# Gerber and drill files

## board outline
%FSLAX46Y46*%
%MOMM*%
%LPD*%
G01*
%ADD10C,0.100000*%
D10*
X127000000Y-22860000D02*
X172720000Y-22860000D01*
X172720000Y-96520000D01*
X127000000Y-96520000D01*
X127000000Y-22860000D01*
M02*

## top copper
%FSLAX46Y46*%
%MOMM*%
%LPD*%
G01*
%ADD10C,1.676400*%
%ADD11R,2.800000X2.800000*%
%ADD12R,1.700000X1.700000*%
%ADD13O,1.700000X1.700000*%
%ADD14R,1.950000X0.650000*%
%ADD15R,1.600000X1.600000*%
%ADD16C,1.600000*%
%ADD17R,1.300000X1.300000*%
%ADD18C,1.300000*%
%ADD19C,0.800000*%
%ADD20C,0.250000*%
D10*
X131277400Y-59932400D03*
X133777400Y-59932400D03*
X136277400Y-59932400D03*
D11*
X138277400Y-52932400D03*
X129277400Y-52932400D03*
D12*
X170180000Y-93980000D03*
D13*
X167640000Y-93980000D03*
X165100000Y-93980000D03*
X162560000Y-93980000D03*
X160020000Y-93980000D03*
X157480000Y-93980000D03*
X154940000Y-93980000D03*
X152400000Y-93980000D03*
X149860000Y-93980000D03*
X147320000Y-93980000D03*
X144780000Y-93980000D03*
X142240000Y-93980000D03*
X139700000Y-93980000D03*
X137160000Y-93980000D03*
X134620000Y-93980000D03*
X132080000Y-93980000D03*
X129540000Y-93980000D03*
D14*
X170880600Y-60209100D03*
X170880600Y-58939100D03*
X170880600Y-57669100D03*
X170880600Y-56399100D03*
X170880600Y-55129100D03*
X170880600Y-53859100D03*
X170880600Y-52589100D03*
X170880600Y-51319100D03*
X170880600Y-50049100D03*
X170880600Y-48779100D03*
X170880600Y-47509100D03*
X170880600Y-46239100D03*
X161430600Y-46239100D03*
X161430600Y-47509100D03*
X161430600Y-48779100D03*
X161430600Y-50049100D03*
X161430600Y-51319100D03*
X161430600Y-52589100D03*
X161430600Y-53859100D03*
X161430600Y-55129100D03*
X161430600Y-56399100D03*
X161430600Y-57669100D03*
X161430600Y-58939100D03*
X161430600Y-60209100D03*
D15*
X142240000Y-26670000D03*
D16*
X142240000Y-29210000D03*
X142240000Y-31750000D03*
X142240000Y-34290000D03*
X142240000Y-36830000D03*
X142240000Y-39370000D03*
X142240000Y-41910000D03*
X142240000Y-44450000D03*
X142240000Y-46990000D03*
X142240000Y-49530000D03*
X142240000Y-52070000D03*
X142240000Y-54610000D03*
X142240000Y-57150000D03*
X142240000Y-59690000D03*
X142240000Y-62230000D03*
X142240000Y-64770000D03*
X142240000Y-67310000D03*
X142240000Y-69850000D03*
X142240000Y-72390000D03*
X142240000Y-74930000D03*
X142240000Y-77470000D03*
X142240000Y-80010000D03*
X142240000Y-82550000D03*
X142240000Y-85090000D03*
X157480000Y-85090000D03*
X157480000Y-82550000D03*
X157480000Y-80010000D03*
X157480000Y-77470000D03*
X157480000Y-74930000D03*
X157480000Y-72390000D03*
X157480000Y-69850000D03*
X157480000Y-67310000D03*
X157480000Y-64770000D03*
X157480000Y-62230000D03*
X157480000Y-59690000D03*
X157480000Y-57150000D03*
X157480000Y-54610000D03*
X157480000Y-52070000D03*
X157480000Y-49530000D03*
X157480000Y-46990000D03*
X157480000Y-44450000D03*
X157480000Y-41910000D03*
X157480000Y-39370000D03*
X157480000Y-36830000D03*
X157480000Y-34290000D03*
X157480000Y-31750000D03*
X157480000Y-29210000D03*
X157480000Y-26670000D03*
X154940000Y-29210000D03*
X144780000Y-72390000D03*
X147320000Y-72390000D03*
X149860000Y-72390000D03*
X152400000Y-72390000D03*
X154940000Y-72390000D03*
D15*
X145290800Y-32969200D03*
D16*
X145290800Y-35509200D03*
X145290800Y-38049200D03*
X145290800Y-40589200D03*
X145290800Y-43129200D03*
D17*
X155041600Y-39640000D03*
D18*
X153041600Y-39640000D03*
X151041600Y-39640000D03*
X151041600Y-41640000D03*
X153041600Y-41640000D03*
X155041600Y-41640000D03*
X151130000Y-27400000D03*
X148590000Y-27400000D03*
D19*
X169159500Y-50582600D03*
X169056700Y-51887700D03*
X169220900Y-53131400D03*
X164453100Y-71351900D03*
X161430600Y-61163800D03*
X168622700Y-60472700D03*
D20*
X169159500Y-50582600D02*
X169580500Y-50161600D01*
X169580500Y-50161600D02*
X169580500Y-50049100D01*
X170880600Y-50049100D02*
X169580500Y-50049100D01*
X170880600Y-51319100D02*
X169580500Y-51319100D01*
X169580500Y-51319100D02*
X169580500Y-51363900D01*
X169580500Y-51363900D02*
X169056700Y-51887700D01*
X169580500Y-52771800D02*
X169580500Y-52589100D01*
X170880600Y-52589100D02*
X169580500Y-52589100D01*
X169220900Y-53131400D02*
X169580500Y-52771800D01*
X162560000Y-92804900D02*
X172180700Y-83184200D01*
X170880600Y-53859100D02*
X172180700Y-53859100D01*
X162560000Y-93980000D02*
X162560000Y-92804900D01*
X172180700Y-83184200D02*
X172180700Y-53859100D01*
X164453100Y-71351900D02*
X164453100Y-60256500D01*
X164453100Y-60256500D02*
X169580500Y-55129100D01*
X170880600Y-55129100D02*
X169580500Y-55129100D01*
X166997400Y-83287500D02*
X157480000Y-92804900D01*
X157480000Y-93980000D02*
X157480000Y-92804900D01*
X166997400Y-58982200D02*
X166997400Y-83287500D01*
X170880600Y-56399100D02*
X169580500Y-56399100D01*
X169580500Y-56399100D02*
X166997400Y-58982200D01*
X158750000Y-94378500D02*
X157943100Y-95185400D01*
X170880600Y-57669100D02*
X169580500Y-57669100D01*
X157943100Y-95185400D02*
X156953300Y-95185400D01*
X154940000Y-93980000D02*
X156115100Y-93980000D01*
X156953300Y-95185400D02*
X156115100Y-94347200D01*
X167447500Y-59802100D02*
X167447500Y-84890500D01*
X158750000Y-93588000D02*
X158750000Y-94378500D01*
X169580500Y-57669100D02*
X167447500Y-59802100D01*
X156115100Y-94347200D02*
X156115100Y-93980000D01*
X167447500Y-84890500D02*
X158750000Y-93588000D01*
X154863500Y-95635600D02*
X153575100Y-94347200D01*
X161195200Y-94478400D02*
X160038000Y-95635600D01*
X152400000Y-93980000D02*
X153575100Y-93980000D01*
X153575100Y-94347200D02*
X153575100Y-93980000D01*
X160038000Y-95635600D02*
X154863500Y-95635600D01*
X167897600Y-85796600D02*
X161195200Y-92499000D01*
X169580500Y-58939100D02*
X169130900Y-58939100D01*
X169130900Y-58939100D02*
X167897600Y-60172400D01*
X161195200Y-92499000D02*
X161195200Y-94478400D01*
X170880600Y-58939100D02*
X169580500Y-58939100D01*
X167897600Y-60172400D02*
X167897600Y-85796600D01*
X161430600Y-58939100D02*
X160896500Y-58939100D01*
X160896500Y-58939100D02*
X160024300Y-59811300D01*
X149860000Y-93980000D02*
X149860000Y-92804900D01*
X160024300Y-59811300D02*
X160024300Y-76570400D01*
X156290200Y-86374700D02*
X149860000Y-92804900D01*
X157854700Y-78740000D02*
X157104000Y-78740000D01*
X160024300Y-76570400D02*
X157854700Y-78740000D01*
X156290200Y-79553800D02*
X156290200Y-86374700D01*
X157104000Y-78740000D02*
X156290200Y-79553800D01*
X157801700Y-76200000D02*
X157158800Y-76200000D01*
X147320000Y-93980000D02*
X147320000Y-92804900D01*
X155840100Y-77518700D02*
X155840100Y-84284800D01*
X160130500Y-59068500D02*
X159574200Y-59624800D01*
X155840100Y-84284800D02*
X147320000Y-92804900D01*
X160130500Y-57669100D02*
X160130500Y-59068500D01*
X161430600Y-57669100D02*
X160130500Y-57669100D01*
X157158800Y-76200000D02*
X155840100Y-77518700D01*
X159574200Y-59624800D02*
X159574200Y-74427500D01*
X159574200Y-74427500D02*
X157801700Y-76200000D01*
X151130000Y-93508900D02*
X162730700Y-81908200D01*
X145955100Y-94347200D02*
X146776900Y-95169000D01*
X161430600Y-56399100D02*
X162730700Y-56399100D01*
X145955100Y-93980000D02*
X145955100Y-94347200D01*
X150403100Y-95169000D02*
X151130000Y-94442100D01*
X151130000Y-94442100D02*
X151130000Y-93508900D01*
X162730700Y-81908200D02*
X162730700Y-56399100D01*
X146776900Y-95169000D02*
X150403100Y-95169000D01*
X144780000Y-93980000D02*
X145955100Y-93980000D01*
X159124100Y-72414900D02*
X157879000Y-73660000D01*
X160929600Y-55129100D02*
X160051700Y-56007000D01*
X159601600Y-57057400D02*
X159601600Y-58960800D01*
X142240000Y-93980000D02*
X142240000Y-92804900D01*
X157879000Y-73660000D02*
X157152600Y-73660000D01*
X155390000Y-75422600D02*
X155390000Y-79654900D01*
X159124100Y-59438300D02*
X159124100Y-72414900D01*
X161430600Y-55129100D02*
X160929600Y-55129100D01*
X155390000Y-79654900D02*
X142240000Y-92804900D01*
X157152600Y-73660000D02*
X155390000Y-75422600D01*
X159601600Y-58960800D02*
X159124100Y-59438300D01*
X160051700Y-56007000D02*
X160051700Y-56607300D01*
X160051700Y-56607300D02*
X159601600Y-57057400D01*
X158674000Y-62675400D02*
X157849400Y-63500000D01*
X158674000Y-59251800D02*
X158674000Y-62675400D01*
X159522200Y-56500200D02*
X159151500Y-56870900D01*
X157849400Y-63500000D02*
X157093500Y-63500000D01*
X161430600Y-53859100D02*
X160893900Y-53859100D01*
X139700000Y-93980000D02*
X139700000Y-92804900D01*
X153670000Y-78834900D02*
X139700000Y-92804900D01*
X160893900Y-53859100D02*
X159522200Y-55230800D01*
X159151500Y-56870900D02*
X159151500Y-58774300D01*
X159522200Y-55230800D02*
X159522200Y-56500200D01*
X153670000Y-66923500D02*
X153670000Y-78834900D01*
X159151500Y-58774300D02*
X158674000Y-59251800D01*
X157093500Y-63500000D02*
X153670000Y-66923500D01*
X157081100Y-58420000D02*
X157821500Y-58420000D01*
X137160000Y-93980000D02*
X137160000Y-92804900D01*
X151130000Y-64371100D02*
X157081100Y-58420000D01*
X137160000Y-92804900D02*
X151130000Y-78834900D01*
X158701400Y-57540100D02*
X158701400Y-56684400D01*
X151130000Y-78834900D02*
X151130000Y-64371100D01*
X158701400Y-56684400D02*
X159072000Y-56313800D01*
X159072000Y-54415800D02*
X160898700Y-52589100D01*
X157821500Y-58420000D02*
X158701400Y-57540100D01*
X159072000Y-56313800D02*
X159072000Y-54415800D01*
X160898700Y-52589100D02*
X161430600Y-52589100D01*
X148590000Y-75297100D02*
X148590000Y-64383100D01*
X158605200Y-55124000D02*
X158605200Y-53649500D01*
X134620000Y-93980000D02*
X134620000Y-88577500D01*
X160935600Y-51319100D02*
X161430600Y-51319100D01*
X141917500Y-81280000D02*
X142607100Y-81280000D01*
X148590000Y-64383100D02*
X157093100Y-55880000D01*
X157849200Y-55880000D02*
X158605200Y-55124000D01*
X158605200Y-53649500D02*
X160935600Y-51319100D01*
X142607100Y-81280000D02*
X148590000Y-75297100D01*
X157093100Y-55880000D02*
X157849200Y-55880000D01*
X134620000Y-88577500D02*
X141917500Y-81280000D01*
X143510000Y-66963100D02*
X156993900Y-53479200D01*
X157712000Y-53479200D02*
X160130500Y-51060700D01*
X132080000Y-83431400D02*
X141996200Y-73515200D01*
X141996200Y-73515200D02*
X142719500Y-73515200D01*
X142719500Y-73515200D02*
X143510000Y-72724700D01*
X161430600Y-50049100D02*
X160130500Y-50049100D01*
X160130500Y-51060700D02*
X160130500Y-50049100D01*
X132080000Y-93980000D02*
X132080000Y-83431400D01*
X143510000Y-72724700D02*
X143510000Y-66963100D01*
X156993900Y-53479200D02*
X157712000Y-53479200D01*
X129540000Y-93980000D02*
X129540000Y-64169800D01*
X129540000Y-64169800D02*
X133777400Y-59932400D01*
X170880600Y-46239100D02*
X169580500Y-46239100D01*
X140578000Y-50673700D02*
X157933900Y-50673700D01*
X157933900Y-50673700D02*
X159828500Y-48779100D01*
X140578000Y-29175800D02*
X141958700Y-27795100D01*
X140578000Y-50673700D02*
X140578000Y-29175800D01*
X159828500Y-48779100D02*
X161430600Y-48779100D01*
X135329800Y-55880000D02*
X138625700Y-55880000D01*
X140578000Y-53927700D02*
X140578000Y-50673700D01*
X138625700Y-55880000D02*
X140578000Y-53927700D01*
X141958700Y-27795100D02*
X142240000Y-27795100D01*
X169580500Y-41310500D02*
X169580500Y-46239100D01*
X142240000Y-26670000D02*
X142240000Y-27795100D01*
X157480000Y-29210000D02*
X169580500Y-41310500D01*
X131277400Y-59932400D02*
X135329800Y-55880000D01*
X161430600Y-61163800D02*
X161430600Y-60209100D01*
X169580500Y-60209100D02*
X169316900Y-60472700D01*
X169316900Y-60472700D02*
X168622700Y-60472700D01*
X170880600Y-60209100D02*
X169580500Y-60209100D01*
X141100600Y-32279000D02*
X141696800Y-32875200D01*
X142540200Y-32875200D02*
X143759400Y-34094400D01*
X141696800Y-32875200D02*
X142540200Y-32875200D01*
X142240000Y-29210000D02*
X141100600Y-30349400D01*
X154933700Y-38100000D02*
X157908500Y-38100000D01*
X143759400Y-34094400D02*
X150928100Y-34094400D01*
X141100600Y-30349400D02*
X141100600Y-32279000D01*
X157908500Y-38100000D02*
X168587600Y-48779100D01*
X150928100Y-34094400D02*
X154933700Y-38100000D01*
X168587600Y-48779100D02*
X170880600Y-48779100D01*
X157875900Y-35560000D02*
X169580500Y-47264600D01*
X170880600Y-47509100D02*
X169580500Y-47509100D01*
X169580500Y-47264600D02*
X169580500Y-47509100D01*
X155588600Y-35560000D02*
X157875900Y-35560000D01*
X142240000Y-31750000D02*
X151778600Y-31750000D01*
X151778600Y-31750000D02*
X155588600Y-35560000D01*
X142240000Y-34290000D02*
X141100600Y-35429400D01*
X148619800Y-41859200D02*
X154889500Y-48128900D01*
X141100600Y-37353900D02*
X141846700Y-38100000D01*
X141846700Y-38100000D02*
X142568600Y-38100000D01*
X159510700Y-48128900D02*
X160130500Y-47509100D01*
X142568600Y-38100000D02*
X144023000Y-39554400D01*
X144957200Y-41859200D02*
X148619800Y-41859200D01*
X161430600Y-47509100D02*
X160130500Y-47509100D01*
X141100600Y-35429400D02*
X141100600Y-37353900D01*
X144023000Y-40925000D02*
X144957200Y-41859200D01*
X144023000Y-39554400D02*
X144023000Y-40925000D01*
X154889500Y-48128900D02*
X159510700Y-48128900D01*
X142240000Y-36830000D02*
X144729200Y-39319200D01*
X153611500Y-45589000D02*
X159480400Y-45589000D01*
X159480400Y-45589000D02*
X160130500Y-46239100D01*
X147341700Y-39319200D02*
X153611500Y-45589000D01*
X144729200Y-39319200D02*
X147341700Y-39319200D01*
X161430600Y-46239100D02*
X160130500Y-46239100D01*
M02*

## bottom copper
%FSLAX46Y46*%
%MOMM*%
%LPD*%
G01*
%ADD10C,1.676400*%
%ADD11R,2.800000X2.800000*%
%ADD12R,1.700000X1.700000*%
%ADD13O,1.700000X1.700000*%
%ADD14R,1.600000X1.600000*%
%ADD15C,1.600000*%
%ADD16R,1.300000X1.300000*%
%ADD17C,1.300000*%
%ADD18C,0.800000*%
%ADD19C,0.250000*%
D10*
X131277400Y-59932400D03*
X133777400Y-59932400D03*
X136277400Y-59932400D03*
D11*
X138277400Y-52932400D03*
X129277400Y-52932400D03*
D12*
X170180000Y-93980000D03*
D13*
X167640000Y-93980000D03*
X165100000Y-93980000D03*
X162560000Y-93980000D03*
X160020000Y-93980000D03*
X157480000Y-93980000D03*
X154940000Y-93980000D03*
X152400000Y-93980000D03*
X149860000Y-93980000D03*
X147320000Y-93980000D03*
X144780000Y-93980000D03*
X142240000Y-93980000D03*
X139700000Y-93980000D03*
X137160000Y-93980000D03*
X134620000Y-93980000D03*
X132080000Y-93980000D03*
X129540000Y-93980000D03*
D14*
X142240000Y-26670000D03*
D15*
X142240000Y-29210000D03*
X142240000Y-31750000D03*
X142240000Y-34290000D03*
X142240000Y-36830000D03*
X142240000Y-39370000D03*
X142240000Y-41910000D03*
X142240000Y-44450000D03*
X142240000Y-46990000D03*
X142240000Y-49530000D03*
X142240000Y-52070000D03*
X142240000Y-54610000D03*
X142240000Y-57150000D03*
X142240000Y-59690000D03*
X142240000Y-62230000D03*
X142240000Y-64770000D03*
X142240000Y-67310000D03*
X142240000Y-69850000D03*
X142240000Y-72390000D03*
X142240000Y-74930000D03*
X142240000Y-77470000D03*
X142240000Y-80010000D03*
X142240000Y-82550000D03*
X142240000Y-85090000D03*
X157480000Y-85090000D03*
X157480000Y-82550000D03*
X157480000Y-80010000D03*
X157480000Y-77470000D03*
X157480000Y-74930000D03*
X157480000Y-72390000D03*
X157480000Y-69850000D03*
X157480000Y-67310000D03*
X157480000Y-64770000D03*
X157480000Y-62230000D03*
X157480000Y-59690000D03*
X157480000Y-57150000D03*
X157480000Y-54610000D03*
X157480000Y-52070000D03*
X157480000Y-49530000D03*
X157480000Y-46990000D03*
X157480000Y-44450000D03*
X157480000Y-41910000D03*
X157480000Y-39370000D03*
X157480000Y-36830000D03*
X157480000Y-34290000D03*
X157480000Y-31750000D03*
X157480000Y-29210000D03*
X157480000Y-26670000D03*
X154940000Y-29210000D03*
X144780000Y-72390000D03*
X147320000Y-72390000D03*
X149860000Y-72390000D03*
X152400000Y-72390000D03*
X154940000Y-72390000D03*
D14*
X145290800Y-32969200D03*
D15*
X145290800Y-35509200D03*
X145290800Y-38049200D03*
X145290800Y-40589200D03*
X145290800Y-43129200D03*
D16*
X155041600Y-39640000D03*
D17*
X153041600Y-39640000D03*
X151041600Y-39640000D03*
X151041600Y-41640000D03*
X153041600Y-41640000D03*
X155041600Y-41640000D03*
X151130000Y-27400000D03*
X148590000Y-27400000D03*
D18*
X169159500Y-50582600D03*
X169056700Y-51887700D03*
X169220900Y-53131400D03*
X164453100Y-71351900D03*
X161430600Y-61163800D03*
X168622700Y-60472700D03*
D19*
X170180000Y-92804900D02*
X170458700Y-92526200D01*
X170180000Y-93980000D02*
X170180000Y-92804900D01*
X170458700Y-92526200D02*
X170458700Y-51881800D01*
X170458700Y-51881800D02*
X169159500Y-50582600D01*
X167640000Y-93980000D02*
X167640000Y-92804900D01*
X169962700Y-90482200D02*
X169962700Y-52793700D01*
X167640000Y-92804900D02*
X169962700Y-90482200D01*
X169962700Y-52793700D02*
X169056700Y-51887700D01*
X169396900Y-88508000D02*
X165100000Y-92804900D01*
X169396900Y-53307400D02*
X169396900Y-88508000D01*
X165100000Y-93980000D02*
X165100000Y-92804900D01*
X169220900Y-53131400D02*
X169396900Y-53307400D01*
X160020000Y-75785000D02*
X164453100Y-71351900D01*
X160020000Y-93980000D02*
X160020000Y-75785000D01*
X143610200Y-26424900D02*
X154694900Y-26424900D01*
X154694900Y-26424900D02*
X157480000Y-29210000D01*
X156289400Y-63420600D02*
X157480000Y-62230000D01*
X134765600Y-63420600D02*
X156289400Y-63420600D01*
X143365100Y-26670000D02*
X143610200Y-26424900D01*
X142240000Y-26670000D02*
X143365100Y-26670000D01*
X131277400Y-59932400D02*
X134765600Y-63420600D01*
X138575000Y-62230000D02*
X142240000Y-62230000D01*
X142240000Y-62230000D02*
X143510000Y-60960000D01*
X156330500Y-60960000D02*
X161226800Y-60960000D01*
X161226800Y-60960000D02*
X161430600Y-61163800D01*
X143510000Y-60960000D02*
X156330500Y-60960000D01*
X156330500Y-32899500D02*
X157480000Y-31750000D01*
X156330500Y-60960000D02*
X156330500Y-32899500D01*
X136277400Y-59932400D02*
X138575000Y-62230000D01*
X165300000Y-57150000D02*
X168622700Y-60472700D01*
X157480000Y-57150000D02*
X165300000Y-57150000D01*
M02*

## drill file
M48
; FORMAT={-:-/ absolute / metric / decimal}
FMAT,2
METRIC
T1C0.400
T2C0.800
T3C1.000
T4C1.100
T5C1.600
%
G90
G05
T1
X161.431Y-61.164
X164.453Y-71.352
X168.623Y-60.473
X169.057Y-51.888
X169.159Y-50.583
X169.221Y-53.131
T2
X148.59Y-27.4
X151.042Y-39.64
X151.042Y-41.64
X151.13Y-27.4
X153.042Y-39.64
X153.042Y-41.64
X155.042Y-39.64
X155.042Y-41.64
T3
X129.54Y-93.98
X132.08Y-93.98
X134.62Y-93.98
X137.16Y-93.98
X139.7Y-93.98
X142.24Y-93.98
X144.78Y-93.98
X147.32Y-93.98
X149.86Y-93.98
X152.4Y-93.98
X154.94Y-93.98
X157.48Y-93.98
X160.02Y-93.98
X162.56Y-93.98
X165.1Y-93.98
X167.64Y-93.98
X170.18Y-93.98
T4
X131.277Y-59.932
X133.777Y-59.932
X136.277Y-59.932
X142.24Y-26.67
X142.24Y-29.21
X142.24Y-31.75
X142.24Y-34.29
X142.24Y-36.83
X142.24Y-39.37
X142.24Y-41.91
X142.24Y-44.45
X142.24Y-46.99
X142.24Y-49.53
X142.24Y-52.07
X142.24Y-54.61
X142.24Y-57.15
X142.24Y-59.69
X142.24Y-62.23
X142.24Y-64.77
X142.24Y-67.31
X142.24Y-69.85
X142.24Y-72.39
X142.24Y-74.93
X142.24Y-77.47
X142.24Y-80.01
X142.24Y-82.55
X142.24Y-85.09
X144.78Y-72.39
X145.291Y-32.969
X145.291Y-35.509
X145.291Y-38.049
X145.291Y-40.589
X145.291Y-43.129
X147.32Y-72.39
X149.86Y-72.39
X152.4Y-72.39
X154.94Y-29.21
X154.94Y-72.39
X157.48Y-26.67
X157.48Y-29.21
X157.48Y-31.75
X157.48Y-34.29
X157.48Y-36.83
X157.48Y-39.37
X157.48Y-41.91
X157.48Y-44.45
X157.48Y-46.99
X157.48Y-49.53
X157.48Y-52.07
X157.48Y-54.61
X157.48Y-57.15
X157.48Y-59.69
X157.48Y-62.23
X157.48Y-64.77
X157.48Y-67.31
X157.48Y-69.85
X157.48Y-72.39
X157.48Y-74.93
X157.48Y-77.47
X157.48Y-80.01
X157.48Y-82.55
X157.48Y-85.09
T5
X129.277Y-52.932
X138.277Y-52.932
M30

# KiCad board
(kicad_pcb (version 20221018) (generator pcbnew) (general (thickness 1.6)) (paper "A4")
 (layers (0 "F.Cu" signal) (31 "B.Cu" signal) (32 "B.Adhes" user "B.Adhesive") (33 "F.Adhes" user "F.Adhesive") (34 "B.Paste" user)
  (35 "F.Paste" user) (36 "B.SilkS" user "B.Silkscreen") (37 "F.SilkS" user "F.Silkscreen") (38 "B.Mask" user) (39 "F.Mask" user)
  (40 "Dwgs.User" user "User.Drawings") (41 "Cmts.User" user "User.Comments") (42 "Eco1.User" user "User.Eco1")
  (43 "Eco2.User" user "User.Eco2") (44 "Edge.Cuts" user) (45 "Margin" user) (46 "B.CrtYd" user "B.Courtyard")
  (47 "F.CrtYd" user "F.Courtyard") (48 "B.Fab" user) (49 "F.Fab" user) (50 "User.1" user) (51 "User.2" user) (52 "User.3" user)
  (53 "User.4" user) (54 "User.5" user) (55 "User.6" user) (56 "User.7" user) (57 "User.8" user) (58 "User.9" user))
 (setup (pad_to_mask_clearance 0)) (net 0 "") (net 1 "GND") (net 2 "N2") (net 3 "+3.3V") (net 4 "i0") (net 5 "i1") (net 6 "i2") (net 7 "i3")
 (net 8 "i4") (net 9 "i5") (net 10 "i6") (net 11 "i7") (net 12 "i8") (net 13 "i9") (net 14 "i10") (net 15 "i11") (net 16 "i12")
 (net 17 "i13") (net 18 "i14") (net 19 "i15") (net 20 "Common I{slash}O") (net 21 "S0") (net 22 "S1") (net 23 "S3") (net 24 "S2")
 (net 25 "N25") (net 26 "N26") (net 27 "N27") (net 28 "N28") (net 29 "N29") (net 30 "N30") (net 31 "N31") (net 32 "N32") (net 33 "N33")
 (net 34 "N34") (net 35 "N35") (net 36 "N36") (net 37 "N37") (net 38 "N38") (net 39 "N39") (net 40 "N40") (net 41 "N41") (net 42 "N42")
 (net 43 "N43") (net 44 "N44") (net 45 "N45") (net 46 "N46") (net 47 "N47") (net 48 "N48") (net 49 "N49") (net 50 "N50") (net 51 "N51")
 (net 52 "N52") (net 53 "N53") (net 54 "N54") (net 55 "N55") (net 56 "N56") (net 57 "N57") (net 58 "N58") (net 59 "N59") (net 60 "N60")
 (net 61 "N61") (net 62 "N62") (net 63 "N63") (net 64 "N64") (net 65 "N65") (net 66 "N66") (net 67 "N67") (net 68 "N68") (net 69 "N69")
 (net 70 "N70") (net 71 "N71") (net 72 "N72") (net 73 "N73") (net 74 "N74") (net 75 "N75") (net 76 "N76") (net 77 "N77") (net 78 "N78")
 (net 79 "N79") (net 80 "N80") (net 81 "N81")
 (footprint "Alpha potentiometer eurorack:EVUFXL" (layer "F.Cu") (at 133.7774 52.9324)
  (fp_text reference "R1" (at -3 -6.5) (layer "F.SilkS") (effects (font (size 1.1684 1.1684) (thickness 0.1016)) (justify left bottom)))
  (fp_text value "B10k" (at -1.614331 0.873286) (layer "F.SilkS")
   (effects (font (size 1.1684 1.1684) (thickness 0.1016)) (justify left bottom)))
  (pad "1" thru_hole circle (at -2.5 7 270) (size 1.6764 1.6764) (drill 1.1) (layers "*.Cu" "*.Mask") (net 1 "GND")
   (solder_mask_margin 0.1016))
  (pad "2" thru_hole circle (at 0 7 270) (size 1.6764 1.6764) (drill 1.1) (layers "*.Cu" "*.Mask") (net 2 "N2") (solder_mask_margin 0.1016))
  (pad "3" thru_hole circle (at 2.5 7 270) (size 1.6764 1.6764) (drill 1.1) (layers "*.Cu" "*.Mask") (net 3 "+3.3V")
   (solder_mask_margin 0.1016))
  (pad "M1" thru_hole rect (at 4.5 0 270) (size 2.8 2.8) (drill 1.6) (layers "*.Cu" "*.Mask") (solder_mask_margin 0.1016)
   (thermal_bridge_angle 45))
  (pad "M2" thru_hole rect (at -4.5 0 270) (size 2.8 2.8) (drill 1.6) (layers "*.Cu" "*.Mask") (solder_mask_margin 0.1016)
   (thermal_bridge_angle 45)))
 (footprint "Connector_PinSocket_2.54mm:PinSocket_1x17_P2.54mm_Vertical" (layer "F.Cu") (at 170.18 93.98 -90)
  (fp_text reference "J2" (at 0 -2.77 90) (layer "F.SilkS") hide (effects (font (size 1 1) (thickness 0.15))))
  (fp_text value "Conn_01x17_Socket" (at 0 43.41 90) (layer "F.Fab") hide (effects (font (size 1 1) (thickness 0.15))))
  (pad "1" thru_hole rect (at 0 0 270) (size 1.7 1.7) (drill 1) (layers "*.Cu" "*.Mask") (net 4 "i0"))
  (pad "2" thru_hole oval (at 0 2.54 270) (size 1.7 1.7) (drill 1) (layers "*.Cu" "*.Mask") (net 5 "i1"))
  (pad "3" thru_hole oval (at 0 5.08 270) (size 1.7 1.7) (drill 1) (layers "*.Cu" "*.Mask") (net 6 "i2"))
  (pad "4" thru_hole oval (at 0 7.62 270) (size 1.7 1.7) (drill 1) (layers "*.Cu" "*.Mask") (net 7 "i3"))
  (pad "5" thru_hole oval (at 0 10.16 270) (size 1.7 1.7) (drill 1) (layers "*.Cu" "*.Mask") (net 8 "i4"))
  (pad "6" thru_hole oval (at 0 12.7 270) (size 1.7 1.7) (drill 1) (layers "*.Cu" "*.Mask") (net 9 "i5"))
  (pad "7" thru_hole oval (at 0 15.24 270) (size 1.7 1.7) (drill 1) (layers "*.Cu" "*.Mask") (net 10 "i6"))
  (pad "8" thru_hole oval (at 0 17.78 270) (size 1.7 1.7) (drill 1) (layers "*.Cu" "*.Mask") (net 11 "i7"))
  (pad "9" thru_hole oval (at 0 20.32 270) (size 1.7 1.7) (drill 1) (layers "*.Cu" "*.Mask") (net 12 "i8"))
  (pad "10" thru_hole oval (at 0 22.86 270) (size 1.7 1.7) (drill 1) (layers "*.Cu" "*.Mask") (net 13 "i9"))
  (pad "11" thru_hole oval (at 0 25.4 270) (size 1.7 1.7) (drill 1) (layers "*.Cu" "*.Mask") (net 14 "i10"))
  (pad "12" thru_hole oval (at 0 27.94 270) (size 1.7 1.7) (drill 1) (layers "*.Cu" "*.Mask") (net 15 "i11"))
  (pad "13" thru_hole oval (at 0 30.48 270) (size 1.7 1.7) (drill 1) (layers "*.Cu" "*.Mask") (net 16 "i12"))
  (pad "14" thru_hole oval (at 0 33.02 270) (size 1.7 1.7) (drill 1) (layers "*.Cu" "*.Mask") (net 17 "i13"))
  (pad "15" thru_hole oval (at 0 35.56 270) (size 1.7 1.7) (drill 1) (layers "*.Cu" "*.Mask") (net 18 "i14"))
  (pad "16" thru_hole oval (at 0 38.1 270) (size 1.7 1.7) (drill 1) (layers "*.Cu" "*.Mask") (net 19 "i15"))
  (pad "17" thru_hole oval (at 0 40.64 270) (size 1.7 1.7) (drill 1) (layers "*.Cu" "*.Mask") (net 2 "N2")))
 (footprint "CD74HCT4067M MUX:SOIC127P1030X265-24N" (layer "F.Cu") (at 166.1556 53.2241 180)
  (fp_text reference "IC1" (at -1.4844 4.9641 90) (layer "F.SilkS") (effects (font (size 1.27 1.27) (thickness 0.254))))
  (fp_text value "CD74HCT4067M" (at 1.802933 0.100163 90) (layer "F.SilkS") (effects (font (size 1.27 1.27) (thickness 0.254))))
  (pad "1" smd rect (at -4.725 -6.985 270) (size 0.65 1.95) (layers "F.Cu" "F.Paste" "F.Mask") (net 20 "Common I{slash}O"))
  (pad "2" smd rect (at -4.725 -5.715 270) (size 0.65 1.95) (layers "F.Cu" "F.Paste" "F.Mask") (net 11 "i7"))
  (pad "3" smd rect (at -4.725 -4.445 270) (size 0.65 1.95) (layers "F.Cu" "F.Paste" "F.Mask") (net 10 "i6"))
  (pad "4" smd rect (at -4.725 -3.175 270) (size 0.65 1.95) (layers "F.Cu" "F.Paste" "F.Mask") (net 9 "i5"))
  (pad "5" smd rect (at -4.725 -1.905 270) (size 0.65 1.95) (layers "F.Cu" "F.Paste" "F.Mask") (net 8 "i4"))
  (pad "6" smd rect (at -4.725 -0.635 270) (size 0.65 1.95) (layers "F.Cu" "F.Paste" "F.Mask") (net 7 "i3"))
  (pad "7" smd rect (at -4.725 0.635 270) (size 0.65 1.95) (layers "F.Cu" "F.Paste" "F.Mask") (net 6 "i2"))
  (pad "8" smd rect (at -4.725 1.905 270) (size 0.65 1.95) (layers "F.Cu" "F.Paste" "F.Mask") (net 5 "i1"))
  (pad "9" smd rect (at -4.725 3.175 270) (size 0.65 1.95) (layers "F.Cu" "F.Paste" "F.Mask") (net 4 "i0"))
  (pad "10" smd rect (at -4.725 4.445 270) (size 0.65 1.95) (layers "F.Cu" "F.Paste" "F.Mask") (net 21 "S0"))
  (pad "11" smd rect (at -4.725 5.715 270) (size 0.65 1.95) (layers "F.Cu" "F.Paste" "F.Mask") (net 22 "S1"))
  (pad "12" smd rect (at -4.725 6.985 270) (size 0.65 1.95) (layers "F.Cu" "F.Paste" "F.Mask") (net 1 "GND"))
  (pad "13" smd rect (at 4.725 6.985 270) (size 0.65 1.95) (layers "F.Cu" "F.Paste" "F.Mask") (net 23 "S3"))
  (pad "14" smd rect (at 4.725 5.715 270) (size 0.65 1.95) (layers "F.Cu" "F.Paste" "F.Mask") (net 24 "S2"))
  (pad "15" smd rect (at 4.725 4.445 270) (size 0.65 1.95) (layers "F.Cu" "F.Paste" "F.Mask") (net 1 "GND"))
  (pad "16" smd rect (at 4.725 3.175 270) (size 0.65 1.95) (layers "F.Cu" "F.Paste" "F.Mask") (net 19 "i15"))
  (pad "17" smd rect (at 4.725 1.905 270) (size 0.65 1.95) (layers "F.Cu" "F.Paste" "F.Mask") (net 18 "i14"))
  (pad "18" smd rect (at 4.725 0.635 270) (size 0.65 1.95) (layers "F.Cu" "F.Paste" "F.Mask") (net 17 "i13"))
  (pad "19" smd rect (at 4.725 -0.635 270) (size 0.65 1.95) (layers "F.Cu" "F.Paste" "F.Mask") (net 16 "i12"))
  (pad "20" smd rect (at 4.725 -1.905 270) (size 0.65 1.95) (layers "F.Cu" "F.Paste" "F.Mask") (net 15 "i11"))
  (pad "21" smd rect (at 4.725 -3.175 270) (size 0.65 1.95) (layers "F.Cu" "F.Paste" "F.Mask") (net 14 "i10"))
  (pad "22" smd rect (at 4.725 -4.445 270) (size 0.65 1.95) (layers "F.Cu" "F.Paste" "F.Mask") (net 13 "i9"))
  (pad "23" smd rect (at 4.725 -5.715 270) (size 0.65 1.95) (layers "F.Cu" "F.Paste" "F.Mask") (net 12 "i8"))
  (pad "24" smd rect (at 4.725 -6.985 270) (size 0.65 1.95) (layers "F.Cu" "F.Paste" "F.Mask") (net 3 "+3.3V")))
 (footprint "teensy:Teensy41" (layer "F.Cu") (at 149.86 55.88 -90)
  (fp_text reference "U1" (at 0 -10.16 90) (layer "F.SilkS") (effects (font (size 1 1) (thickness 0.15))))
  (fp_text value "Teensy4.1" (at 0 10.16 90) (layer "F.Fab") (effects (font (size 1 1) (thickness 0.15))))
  (pad "1" thru_hole rect (at -29.21 7.62 270) (size 1.6 1.6) (drill 1.1) (layers "*.Cu" "*.Mask") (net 1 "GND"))
  (pad "2" thru_hole circle (at -26.67 7.62 270) (size 1.6 1.6) (drill 1.1) (layers "*.Cu" "*.Mask") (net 21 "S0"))
  (pad "3" thru_hole circle (at -24.13 7.62 270) (size 1.6 1.6) (drill 1.1) (layers "*.Cu" "*.Mask") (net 22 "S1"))
  (pad "4" thru_hole circle (at -21.59 7.62 270) (size 1.6 1.6) (drill 1.1) (layers "*.Cu" "*.Mask") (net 24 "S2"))
  (pad "5" thru_hole circle (at -19.05 7.62 270) (size 1.6 1.6) (drill 1.1) (layers "*.Cu" "*.Mask") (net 23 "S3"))
  (pad "6" thru_hole circle (at -16.51 7.62 270) (size 1.6 1.6) (drill 1.1) (layers "*.Cu" "*.Mask") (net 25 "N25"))
  (pad "7" thru_hole circle (at -13.97 7.62 270) (size 1.6 1.6) (drill 1.1) (layers "*.Cu" "*.Mask") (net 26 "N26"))
  (pad "8" thru_hole circle (at -11.43 7.62 270) (size 1.6 1.6) (drill 1.1) (layers "*.Cu" "*.Mask") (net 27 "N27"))
  (pad "9" thru_hole circle (at -8.89 7.62 270) (size 1.6 1.6) (drill 1.1) (layers "*.Cu" "*.Mask") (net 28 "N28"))
  (pad "10" thru_hole circle (at -6.35 7.62 270) (size 1.6 1.6) (drill 1.1) (layers "*.Cu" "*.Mask") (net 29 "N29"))
  (pad "11" thru_hole circle (at -3.81 7.62 270) (size 1.6 1.6) (drill 1.1) (layers "*.Cu" "*.Mask") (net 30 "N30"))
  (pad "12" thru_hole circle (at -1.27 7.62 270) (size 1.6 1.6) (drill 1.1) (layers "*.Cu" "*.Mask") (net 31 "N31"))
  (pad "13" thru_hole circle (at 1.27 7.62 270) (size 1.6 1.6) (drill 1.1) (layers "*.Cu" "*.Mask") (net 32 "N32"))
  (pad "14" thru_hole circle (at 3.81 7.62 270) (size 1.6 1.6) (drill 1.1) (layers "*.Cu" "*.Mask") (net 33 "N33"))
  (pad "15" thru_hole circle (at 6.35 7.62 270) (size 1.6 1.6) (drill 1.1) (layers "*.Cu" "*.Mask") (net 3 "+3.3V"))
  (pad "16" thru_hole circle (at 8.89 7.62 270) (size 1.6 1.6) (drill 1.1) (layers "*.Cu" "*.Mask") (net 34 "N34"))
  (pad "17" thru_hole circle (at 11.43 7.62 270) (size 1.6 1.6) (drill 1.1) (layers "*.Cu" "*.Mask") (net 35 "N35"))
  (pad "18" thru_hole circle (at 13.97 7.62 270) (size 1.6 1.6) (drill 1.1) (layers "*.Cu" "*.Mask") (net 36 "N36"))
  (pad "19" thru_hole circle (at 16.51 7.62 270) (size 1.6 1.6) (drill 1.1) (layers "*.Cu" "*.Mask") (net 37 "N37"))
  (pad "20" thru_hole circle (at 19.05 7.62 270) (size 1.6 1.6) (drill 1.1) (layers "*.Cu" "*.Mask") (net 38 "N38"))
  (pad "21" thru_hole circle (at 21.59 7.62 270) (size 1.6 1.6) (drill 1.1) (layers "*.Cu" "*.Mask") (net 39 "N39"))
  (pad "22" thru_hole circle (at 24.13 7.62 270) (size 1.6 1.6) (drill 1.1) (layers "*.Cu" "*.Mask") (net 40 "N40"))
  (pad "23" thru_hole circle (at 26.67 7.62 270) (size 1.6 1.6) (drill 1.1) (layers "*.Cu" "*.Mask") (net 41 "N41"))
  (pad "24" thru_hole circle (at 29.21 7.62 270) (size 1.6 1.6) (drill 1.1) (layers "*.Cu" "*.Mask") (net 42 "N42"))
  (pad "25" thru_hole circle (at 29.21 -7.62 270) (size 1.6 1.6) (drill 1.1) (layers "*.Cu" "*.Mask") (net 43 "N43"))
  (pad "26" thru_hole circle (at 26.67 -7.62 270) (size 1.6 1.6) (drill 1.1) (layers "*.Cu" "*.Mask") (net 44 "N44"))
  (pad "27" thru_hole circle (at 24.13 -7.62 270) (size 1.6 1.6) (drill 1.1) (layers "*.Cu" "*.Mask") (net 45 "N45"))
  (pad "28" thru_hole circle (at 21.59 -7.62 270) (size 1.6 1.6) (drill 1.1) (layers "*.Cu" "*.Mask") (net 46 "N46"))
  (pad "29" thru_hole circle (at 19.05 -7.62 270) (size 1.6 1.6) (drill 1.1) (layers "*.Cu" "*.Mask") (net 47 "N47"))
  (pad "30" thru_hole circle (at 16.51 -7.62 270) (size 1.6 1.6) (drill 1.1) (layers "*.Cu" "*.Mask") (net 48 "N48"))
  (pad "31" thru_hole circle (at 13.97 -7.62 270) (size 1.6 1.6) (drill 1.1) (layers "*.Cu" "*.Mask") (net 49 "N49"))
  (pad "32" thru_hole circle (at 11.43 -7.62 270) (size 1.6 1.6) (drill 1.1) (layers "*.Cu" "*.Mask") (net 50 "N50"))
  (pad "33" thru_hole circle (at 8.89 -7.62 270) (size 1.6 1.6) (drill 1.1) (layers "*.Cu" "*.Mask") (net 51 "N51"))
  (pad "34" thru_hole circle (at 6.35 -7.62 270) (size 1.6 1.6) (drill 1.1) (layers "*.Cu" "*.Mask") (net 1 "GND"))
  (pad "35" thru_hole circle (at 3.81 -7.62 270) (size 1.6 1.6) (drill 1.1) (layers "*.Cu" "*.Mask") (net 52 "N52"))
  (pad "36" thru_hole circle (at 1.27 -7.62 270) (size 1.6 1.6) (drill 1.1) (layers "*.Cu" "*.Mask") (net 20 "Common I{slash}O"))
  (pad "37" thru_hole circle (at -1.27 -7.62 270) (size 1.6 1.6) (drill 1.1) (layers "*.Cu" "*.Mask") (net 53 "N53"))
  (pad "38" thru_hole circle (at -3.81 -7.62 270) (size 1.6 1.6) (drill 1.1) (layers "*.Cu" "*.Mask") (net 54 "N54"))
  (pad "39" thru_hole circle (at -6.35 -7.62 270) (size 1.6 1.6) (drill 1.1) (layers "*.Cu" "*.Mask") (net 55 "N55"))
  (pad "40" thru_hole circle (at -8.89 -7.62 270) (size 1.6 1.6) (drill 1.1) (layers "*.Cu" "*.Mask") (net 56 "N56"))
  (pad "41" thru_hole circle (at -11.43 -7.62 270) (size 1.6 1.6) (drill 1.1) (layers "*.Cu" "*.Mask") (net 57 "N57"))
  (pad "42" thru_hole circle (at -13.97 -7.62 270) (size 1.6 1.6) (drill 1.1) (layers "*.Cu" "*.Mask") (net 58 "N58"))
  (pad "43" thru_hole circle (at -16.51 -7.62 270) (size 1.6 1.6) (drill 1.1) (layers "*.Cu" "*.Mask") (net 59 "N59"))
  (pad "44" thru_hole circle (at -19.05 -7.62 270) (size 1.6 1.6) (drill 1.1) (layers "*.Cu" "*.Mask") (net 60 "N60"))
  (pad "45" thru_hole circle (at -21.59 -7.62 270) (size 1.6 1.6) (drill 1.1) (layers "*.Cu" "*.Mask") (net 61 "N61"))
  (pad "46" thru_hole circle (at -24.13 -7.62 270) (size 1.6 1.6) (drill 1.1) (layers "*.Cu" "*.Mask") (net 3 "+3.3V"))
  (pad "47" thru_hole circle (at -26.67 -7.62 270) (size 1.6 1.6) (drill 1.1) (layers "*.Cu" "*.Mask") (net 1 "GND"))
  (pad "48" thru_hole circle (at -29.21 -7.62 270) (size 1.6 1.6) (drill 1.1) (layers "*.Cu" "*.Mask") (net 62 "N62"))
  (pad "49" thru_hole circle (at -26.67 -5.08 270) (size 1.6 1.6) (drill 1.1) (layers "*.Cu" "*.Mask") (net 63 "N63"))
  (pad "50" thru_hole circle (at 16.51 5.08 270) (size 1.6 1.6) (drill 1.1) (layers "*.Cu" "*.Mask") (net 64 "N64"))
  (pad "51" thru_hole circle (at 16.51 2.54 270) (size 1.6 1.6) (drill 1.1) (layers "*.Cu" "*.Mask") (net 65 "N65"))
  (pad "52" thru_hole circle (at 16.51 0 270) (size 1.6 1.6) (drill 1.1) (layers "*.Cu" "*.Mask") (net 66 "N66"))
  (pad "53" thru_hole circle (at 16.51 -2.54 270) (size 1.6 1.6) (drill 1.1) (layers "*.Cu" "*.Mask") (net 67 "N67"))
  (pad "54" thru_hole circle (at 16.51 -5.08 270) (size 1.6 1.6) (drill 1.1) (layers "*.Cu" "*.Mask") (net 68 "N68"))
  (pad "55" thru_hole rect (at -22.9108 4.5692 270) (size 1.6 1.6) (drill 1.1) (layers "*.Cu" "*.Mask") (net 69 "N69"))
  (pad "56" thru_hole circle (at -20.3708 4.5692 270) (size 1.6 1.6) (drill 1.1) (layers "*.Cu" "*.Mask") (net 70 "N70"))
  (pad "57" thru_hole circle (at -17.8308 4.5692 270) (size 1.6 1.6) (drill 1.1) (layers "*.Cu" "*.Mask") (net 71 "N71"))
  (pad "58" thru_hole circle (at -15.2908 4.5692 270) (size 1.6 1.6) (drill 1.1) (layers "*.Cu" "*.Mask") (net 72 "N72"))
  (pad "59" thru_hole circle (at -12.7508 4.5692 270) (size 1.6 1.6) (drill 1.1) (layers "*.Cu" "*.Mask") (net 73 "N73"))
  (pad "60" thru_hole rect (at -16.24 -5.1816 270) (size 1.3 1.3) (drill 0.8) (layers "*.Cu" "*.Mask") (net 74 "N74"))
  (pad "61" thru_hole circle (at -16.24 -3.1816 270) (size 1.3 1.3) (drill 0.8) (layers "*.Cu" "*.Mask") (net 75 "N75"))
  (pad "62" thru_hole circle (at -16.24 -1.1816 270) (size 1.3 1.3) (drill 0.8) (layers "*.Cu" "*.Mask") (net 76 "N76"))
  (pad "63" thru_hole circle (at -14.24 -1.1816 270) (size 1.3 1.3) (drill 0.8) (layers "*.Cu" "*.Mask") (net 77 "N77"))
  (pad "64" thru_hole circle (at -14.24 -3.1816 270) (size 1.3 1.3) (drill 0.8) (layers "*.Cu" "*.Mask") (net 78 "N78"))
  (pad "65" thru_hole circle (at -14.24 -5.1816 270) (size 1.3 1.3) (drill 0.8) (layers "*.Cu" "*.Mask") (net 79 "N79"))
  (pad "66" thru_hole circle (at -28.48 -1.27 270) (size 1.3 1.3) (drill 0.8) (layers "*.Cu" "*.Mask") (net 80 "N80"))
  (pad "67" thru_hole circle (at -28.48 1.27 270) (size 1.3 1.3) (drill 0.8) (layers "*.Cu" "*.Mask") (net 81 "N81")))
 (gr_rect (start 127 22.86) (end 172.72 96.52) (stroke (width 0.1) (type default)) (fill none) (layer "Edge.Cuts"))
 (segment (start 169.1595 50.5826) (end 169.5805 50.1616) (width 0.25) (layer "F.Cu") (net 4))
 (segment (start 169.5805 50.1616) (end 169.5805 50.0491) (width 0.25) (layer "F.Cu") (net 4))
 (segment (start 170.8806 50.0491) (end 169.5805 50.0491) (width 0.25) (layer "F.Cu") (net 4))
 (via (at 169.1595 50.5826) (size 0.8) (drill 0.4) (layers "F.Cu" "B.Cu") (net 4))
 (segment (start 170.18 92.8049) (end 170.4587 92.5262) (width 0.25) (layer "B.Cu") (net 4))
 (segment (start 170.18 93.98) (end 170.18 92.8049) (width 0.25) (layer "B.Cu") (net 4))
 (segment (start 170.4587 92.5262) (end 170.4587 51.8818) (width 0.25) (layer "B.Cu") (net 4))
 (segment (start 170.4587 51.8818) (end 169.1595 50.5826) (width 0.25) (layer "B.Cu") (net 4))
 (segment (start 170.8806 51.3191) (end 169.5805 51.3191) (width 0.25) (layer "F.Cu") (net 5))
 (segment (start 169.5805 51.3191) (end 169.5805 51.3639) (width 0.25) (layer "F.Cu") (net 5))
 (segment (start 169.5805 51.3639) (end 169.0567 51.8877) (width 0.25) (layer "F.Cu") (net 5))
 (via (at 169.0567 51.8877) (size 0.8) (drill 0.4) (layers "F.Cu" "B.Cu") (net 5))
 (segment (start 167.64 93.98) (end 167.64 92.8049) (width 0.25) (layer "B.Cu") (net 5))
 (segment (start 169.9627 90.4822) (end 169.9627 52.7937) (width 0.25) (layer "B.Cu") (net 5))
 (segment (start 167.64 92.8049) (end 169.9627 90.4822) (width 0.25) (layer "B.Cu") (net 5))
 (segment (start 169.9627 52.7937) (end 169.0567 51.8877) (width 0.25) (layer "B.Cu") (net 5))
 (segment (start 169.5805 52.7718) (end 169.5805 52.5891) (width 0.25) (layer "F.Cu") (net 6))
 (segment (start 170.8806 52.5891) (end 169.5805 52.5891) (width 0.25) (layer "F.Cu") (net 6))
 (segment (start 169.2209 53.1314) (end 169.5805 52.7718) (width 0.25) (layer "F.Cu") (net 6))
 (via (at 169.2209 53.1314) (size 0.8) (drill 0.4) (layers "F.Cu" "B.Cu") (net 6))
 (segment (start 169.3969 88.508) (end 165.1 92.8049) (width 0.25) (layer "B.Cu") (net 6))
 (segment (start 169.3969 53.3074) (end 169.3969 88.508) (width 0.25) (layer "B.Cu") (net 6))
 (segment (start 165.1 93.98) (end 165.1 92.8049) (width 0.25) (layer "B.Cu") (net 6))
 (segment (start 169.2209 53.1314) (end 169.3969 53.3074) (width 0.25) (layer "B.Cu") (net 6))
 (segment (start 162.56 92.8049) (end 172.1807 83.1842) (width 0.25) (layer "F.Cu") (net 7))
 (segment (start 170.8806 53.8591) (end 172.1807 53.8591) (width 0.25) (layer "F.Cu") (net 7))
 (segment (start 162.56 93.98) (end 162.56 92.8049) (width 0.25) (layer "F.Cu") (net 7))
 (segment (start 172.1807 83.1842) (end 172.1807 53.8591) (width 0.25) (layer "F.Cu") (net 7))
 (segment (start 164.4531 71.3519) (end 164.4531 60.2565) (width 0.25) (layer "F.Cu") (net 8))
 (segment (start 164.4531 60.2565) (end 169.5805 55.1291) (width 0.25) (layer "F.Cu") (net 8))
 (segment (start 170.8806 55.1291) (end 169.5805 55.1291) (width 0.25) (layer "F.Cu") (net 8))
 (via (at 164.4531 71.3519) (size 0.8) (drill 0.4) (layers "F.Cu" "B.Cu") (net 8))
 (segment (start 160.02 75.785) (end 164.4531 71.3519) (width 0.25) (layer "B.Cu") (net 8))
 (segment (start 160.02 93.98) (end 160.02 75.785) (width 0.25) (layer "B.Cu") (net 8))
 (segment (start 166.9974 83.2875) (end 157.48 92.8049) (width 0.25) (layer "F.Cu") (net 9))
 (segment (start 157.48 93.98) (end 157.48 92.8049) (width 0.25) (layer "F.Cu") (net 9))
 (segment (start 166.9974 58.9822) (end 166.9974 83.2875) (width 0.25) (layer "F.Cu") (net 9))
 (segment (start 170.8806 56.3991) (end 169.5805 56.3991) (width 0.25) (layer "F.Cu") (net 9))
 (segment (start 169.5805 56.3991) (end 166.9974 58.9822) (width 0.25) (layer "F.Cu") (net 9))
 (segment (start 158.75 94.3785) (end 157.9431 95.1854) (width 0.25) (layer "F.Cu") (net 10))
 (segment (start 170.8806 57.6691) (end 169.5805 57.6691) (width 0.25) (layer "F.Cu") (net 10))
 (segment (start 157.9431 95.1854) (end 156.9533 95.1854) (width 0.25) (layer "F.Cu") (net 10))
 (segment (start 154.94 93.98) (end 156.1151 93.98) (width 0.25) (layer "F.Cu") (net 10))
 (segment (start 156.9533 95.1854) (end 156.1151 94.3472) (width 0.25) (layer "F.Cu") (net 10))
 (segment (start 167.4475 59.8021) (end 167.4475 84.8905) (width 0.25) (layer "F.Cu") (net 10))
 (segment (start 158.75 93.588) (end 158.75 94.3785) (width 0.25) (layer "F.Cu") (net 10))
 (segment (start 169.5805 57.6691) (end 167.4475 59.8021) (width 0.25) (layer "F.Cu") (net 10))
 (segment (start 156.1151 94.3472) (end 156.1151 93.98) (width 0.25) (layer "F.Cu") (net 10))
 (segment (start 167.4475 84.8905) (end 158.75 93.588) (width 0.25) (layer "F.Cu") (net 10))
 (segment (start 154.8635 95.6356) (end 153.5751 94.3472) (width 0.25) (layer "F.Cu") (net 11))
 (segment (start 161.1952 94.4784) (end 160.038 95.6356) (width 0.25) (layer "F.Cu") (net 11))
 (segment (start 152.4 93.98) (end 153.5751 93.98) (width 0.25) (layer "F.Cu") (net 11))
 (segment (start 153.5751 94.3472) (end 153.5751 93.98) (width 0.25) (layer "F.Cu") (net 11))
 (segment (start 160.038 95.6356) (end 154.8635 95.6356) (width 0.25) (layer "F.Cu") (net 11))
 (segment (start 167.8976 85.7966) (end 161.1952 92.499) (width 0.25) (layer "F.Cu") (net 11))
 (segment (start 169.5805 58.9391) (end 169.1309 58.9391) (width 0.25) (layer "F.Cu") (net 11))
 (segment (start 169.1309 58.9391) (end 167.8976 60.1724) (width 0.25) (layer "F.Cu") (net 11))
 (segment (start 161.1952 92.499) (end 161.1952 94.4784) (width 0.25) (layer "F.Cu") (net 11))
 (segment (start 170.8806 58.9391) (end 169.5805 58.9391) (width 0.25) (layer "F.Cu") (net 11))
 (segment (start 167.8976 60.1724) (end 167.8976 85.7966) (width 0.25) (layer "F.Cu") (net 11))
 (segment (start 161.4306 58.9391) (end 160.8965 58.9391) (width 0.25) (layer "F.Cu") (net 12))
 (segment (start 160.8965 58.9391) (end 160.0243 59.8113) (width 0.25) (layer "F.Cu") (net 12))
 (segment (start 149.86 93.98) (end 149.86 92.8049) (width 0.25) (layer "F.Cu") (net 12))
 (segment (start 160.0243 59.8113) (end 160.0243 76.5704) (width 0.25) (layer "F.Cu") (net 12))
 (segment (start 156.2902 86.3747) (end 149.86 92.8049) (width 0.25) (layer "F.Cu") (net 12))
 (segment (start 157.8547 78.74) (end 157.104 78.74) (width 0.25) (layer "F.Cu") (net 12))
 (segment (start 160.0243 76.5704) (end 157.8547 78.74) (width 0.25) (layer "F.Cu") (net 12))
 (segment (start 156.2902 79.5538) (end 156.2902 86.3747) (width 0.25) (layer "F.Cu") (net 12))
 (segment (start 157.104 78.74) (end 156.2902 79.5538) (width 0.25) (layer "F.Cu") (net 12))
 (segment (start 157.8017 76.2) (end 157.1588 76.2) (width 0.25) (layer "F.Cu") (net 13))
 (segment (start 147.32 93.98) (end 147.32 92.8049) (width 0.25) (layer "F.Cu") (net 13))
 (segment (start 155.8401 77.5187) (end 155.8401 84.2848) (width 0.25) (layer "F.Cu") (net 13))
 (segment (start 160.1305 59.0685) (end 159.5742 59.6248) (width 0.25) (layer "F.Cu") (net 13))
 (segment (start 155.8401 84.2848) (end 147.32 92.8049) (width 0.25) (layer "F.Cu") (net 13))
 (segment (start 160.1305 57.6691) (end 160.1305 59.0685) (width 0.25) (layer "F.Cu") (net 13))
 (segment (start 161.4306 57.6691) (end 160.1305 57.6691) (width 0.25) (layer "F.Cu") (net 13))
 (segment (start 157.1588 76.2) (end 155.8401 77.5187) (width 0.25) (layer "F.Cu") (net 13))
 (segment (start 159.5742 59.6248) (end 159.5742 74.4275) (width 0.25) (layer "F.Cu") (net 13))
 (segment (start 159.5742 74.4275) (end 157.8017 76.2) (width 0.25) (layer "F.Cu") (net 13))
 (segment (start 151.13 93.5089) (end 162.7307 81.9082) (width 0.25) (layer "F.Cu") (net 14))
 (segment (start 145.9551 94.3472) (end 146.7769 95.169) (width 0.25) (layer "F.Cu") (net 14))
 (segment (start 161.4306 56.3991) (end 162.7307 56.3991) (width 0.25) (layer "F.Cu") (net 14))
 (segment (start 145.9551 93.98) (end 145.9551 94.3472) (width 0.25) (layer "F.Cu") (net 14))
 (segment (start 150.4031 95.169) (end 151.13 94.4421) (width 0.25) (layer "F.Cu") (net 14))
 (segment (start 151.13 94.4421) (end 151.13 93.5089) (width 0.25) (layer "F.Cu") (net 14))
 (segment (start 162.7307 81.9082) (end 162.7307 56.3991) (width 0.25) (layer "F.Cu") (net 14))
 (segment (start 146.7769 95.169) (end 150.4031 95.169) (width 0.25) (layer "F.Cu") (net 14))
 (segment (start 144.78 93.98) (end 145.9551 93.98) (width 0.25) (layer "F.Cu") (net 14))
 (segment (start 159.1241 72.4149) (end 157.879 73.66) (width 0.25) (layer "F.Cu") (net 15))
 (segment (start 160.9296 55.1291) (end 160.0517 56.007) (width 0.25) (layer "F.Cu") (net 15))
 (segment (start 159.6016 57.0574) (end 159.6016 58.9608) (width 0.25) (layer "F.Cu") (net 15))
 (segment (start 142.24 93.98) (end 142.24 92.8049) (width 0.25) (layer "F.Cu") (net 15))
 (segment (start 157.879 73.66) (end 157.1526 73.66) (width 0.25) (layer "F.Cu") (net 15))
 (segment (start 155.39 75.4226) (end 155.39 79.6549) (width 0.25) (layer "F.Cu") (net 15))
 (segment (start 159.1241 59.4383) (end 159.1241 72.4149) (width 0.25) (layer "F.Cu") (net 15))
 (segment (start 161.4306 55.1291) (end 160.9296 55.1291) (width 0.25) (layer "F.Cu") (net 15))
 (segment (start 155.39 79.6549) (end 142.24 92.8049) (width 0.25) (layer "F.Cu") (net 15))
 (segment (start 157.1526 73.66) (end 155.39 75.4226) (width 0.25) (layer "F.Cu") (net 15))
 (segment (start 159.6016 58.9608) (end 159.1241 59.4383) (width 0.25) (layer "F.Cu") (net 15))
 (segment (start 160.0517 56.007) (end 160.0517 56.6073) (width 0.25) (layer "F.Cu") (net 15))
 (segment (start 160.0517 56.6073) (end 159.6016 57.0574) (width 0.25) (layer "F.Cu") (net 15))
 (segment (start 158.674 62.6754) (end 157.8494 63.5) (width 0.25) (layer "F.Cu") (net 16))
 (segment (start 158.674 59.2518) (end 158.674 62.6754) (width 0.25) (layer "F.Cu") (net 16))
 (segment (start 159.5222 56.5002) (end 159.1515 56.8709) (width 0.25) (layer "F.Cu") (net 16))
 (segment (start 157.8494 63.5) (end 157.0935 63.5) (width 0.25) (layer "F.Cu") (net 16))
 (segment (start 161.4306 53.8591) (end 160.8939 53.8591) (width 0.25) (layer "F.Cu") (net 16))
 (segment (start 139.7 93.98) (end 139.7 92.8049) (width 0.25) (layer "F.Cu") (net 16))
 (segment (start 153.67 78.8349) (end 139.7 92.8049) (width 0.25) (layer "F.Cu") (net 16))
 (segment (start 160.8939 53.8591) (end 159.5222 55.2308) (width 0.25) (layer "F.Cu") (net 16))
 (segment (start 159.1515 56.8709) (end 159.1515 58.7743) (width 0.25) (layer "F.Cu") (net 16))
 (segment (start 159.5222 55.2308) (end 159.5222 56.5002) (width 0.25) (layer "F.Cu") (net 16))
 (segment (start 153.67 66.9235) (end 153.67 78.8349) (width 0.25) (layer "F.Cu") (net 16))
 (segment (start 159.1515 58.7743) (end 158.674 59.2518) (width 0.25) (layer "F.Cu") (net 16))
 (segment (start 157.0935 63.5) (end 153.67 66.9235) (width 0.25) (layer "F.Cu") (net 16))
 (segment (start 157.0811 58.42) (end 157.8215 58.42) (width 0.25) (layer "F.Cu") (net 17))
 (segment (start 137.16 93.98) (end 137.16 92.8049) (width 0.25) (layer "F.Cu") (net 17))
 (segment (start 151.13 64.3711) (end 157.0811 58.42) (width 0.25) (layer "F.Cu") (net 17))
 (segment (start 137.16 92.8049) (end 151.13 78.8349) (width 0.25) (layer "F.Cu") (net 17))
 (segment (start 158.7014 57.5401) (end 158.7014 56.6844) (width 0.25) (layer "F.Cu") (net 17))
 (segment (start 151.13 78.8349) (end 151.13 64.3711) (width 0.25) (layer "F.Cu") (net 17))
 (segment (start 158.7014 56.6844) (end 159.072 56.3138) (width 0.25) (layer "F.Cu") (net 17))
 (segment (start 159.072 54.4158) (end 160.8987 52.5891) (width 0.25) (layer "F.Cu") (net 17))
 (segment (start 157.8215 58.42) (end 158.7014 57.5401) (width 0.25) (layer "F.Cu") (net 17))
 (segment (start 159.072 56.3138) (end 159.072 54.4158) (width 0.25) (layer "F.Cu") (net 17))
 (segment (start 160.8987 52.5891) (end 161.4306 52.5891) (width 0.25) (layer "F.Cu") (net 17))
 (segment (start 148.59 75.2971) (end 148.59 64.3831) (width 0.25) (layer "F.Cu") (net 18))
 (segment (start 158.6052 55.124) (end 158.6052 53.6495) (width 0.25) (layer "F.Cu") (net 18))
 (segment (start 134.62 93.98) (end 134.62 88.5775) (width 0.25) (layer "F.Cu") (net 18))
 (segment (start 160.9356 51.3191) (end 161.4306 51.3191) (width 0.25) (layer "F.Cu") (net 18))
 (segment (start 141.9175 81.28) (end 142.6071 81.28) (width 0.25) (layer "F.Cu") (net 18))
 (segment (start 148.59 64.3831) (end 157.0931 55.88) (width 0.25) (layer "F.Cu") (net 18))
 (segment (start 157.8492 55.88) (end 158.6052 55.124) (width 0.25) (layer "F.Cu") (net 18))
 (segment (start 158.6052 53.6495) (end 160.9356 51.3191) (width 0.25) (layer "F.Cu") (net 18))
 (segment (start 142.6071 81.28) (end 148.59 75.2971) (width 0.25) (layer "F.Cu") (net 18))
 (segment (start 157.0931 55.88) (end 157.8492 55.88) (width 0.25) (layer "F.Cu") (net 18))
 (segment (start 134.62 88.5775) (end 141.9175 81.28) (width 0.25) (layer "F.Cu") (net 18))
 (segment (start 143.51 66.9631) (end 156.9939 53.4792) (width 0.25) (layer "F.Cu") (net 19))
 (segment (start 157.712 53.4792) (end 160.1305 51.0607) (width 0.25) (layer "F.Cu") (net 19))
 (segment (start 132.08 83.4314) (end 141.9962 73.5152) (width 0.25) (layer "F.Cu") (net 19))
 (segment (start 141.9962 73.5152) (end 142.7195 73.5152) (width 0.25) (layer "F.Cu") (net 19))
 (segment (start 142.7195 73.5152) (end 143.51 72.7247) (width 0.25) (layer "F.Cu") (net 19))
 (segment (start 161.4306 50.0491) (end 160.1305 50.0491) (width 0.25) (layer "F.Cu") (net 19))
 (segment (start 160.1305 51.0607) (end 160.1305 50.0491) (width 0.25) (layer "F.Cu") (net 19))
 (segment (start 132.08 93.98) (end 132.08 83.4314) (width 0.25) (layer "F.Cu") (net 19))
 (segment (start 143.51 72.7247) (end 143.51 66.9631) (width 0.25) (layer "F.Cu") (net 19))
 (segment (start 156.9939 53.4792) (end 157.712 53.4792) (width 0.25) (layer "F.Cu") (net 19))
 (segment (start 129.54 93.98) (end 129.54 64.1698) (width 0.25) (layer "F.Cu") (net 2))
 (segment (start 129.54 64.1698) (end 133.7774 59.9324) (width 0.25) (layer "F.Cu") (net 2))
 (segment (start 170.8806 46.2391) (end 169.5805 46.2391) (width 0.25) (layer "F.Cu") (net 1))
 (segment (start 140.578 50.6737) (end 157.9339 50.6737) (width 0.25) (layer "F.Cu") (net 1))
 (segment (start 157.9339 50.6737) (end 159.8285 48.7791) (width 0.25) (layer "F.Cu") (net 1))
 (segment (start 140.578 29.1758) (end 141.9587 27.7951) (width 0.25) (layer "F.Cu") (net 1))
 (segment (start 140.578 50.6737) (end 140.578 29.1758) (width 0.25) (layer "F.Cu") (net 1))
 (segment (start 159.8285 48.7791) (end 161.4306 48.7791) (width 0.25) (layer "F.Cu") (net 1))
 (segment (start 135.3298 55.88) (end 138.6257 55.88) (width 0.25) (layer "F.Cu") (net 1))
 (segment (start 140.578 53.9277) (end 140.578 50.6737) (width 0.25) (layer "F.Cu") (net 1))
 (segment (start 138.6257 55.88) (end 140.578 53.9277) (width 0.25) (layer "F.Cu") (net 1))
 (segment (start 141.9587 27.7951) (end 142.24 27.7951) (width 0.25) (layer "F.Cu") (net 1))
 (segment (start 169.5805 41.3105) (end 169.5805 46.2391) (width 0.25) (layer "F.Cu") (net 1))
 (segment (start 142.24 26.67) (end 142.24 27.7951) (width 0.25) (layer "F.Cu") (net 1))
 (segment (start 157.48 29.21) (end 169.5805 41.3105) (width 0.25) (layer "F.Cu") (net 1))
 (segment (start 131.2774 59.9324) (end 135.3298 55.88) (width 0.25) (layer "F.Cu") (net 1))
 (segment (start 143.6102 26.4249) (end 154.6949 26.4249) (width 0.25) (layer "B.Cu") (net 1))
 (segment (start 154.6949 26.4249) (end 157.48 29.21) (width 0.25) (layer "B.Cu") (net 1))
 (segment (start 156.2894 63.4206) (end 157.48 62.23) (width 0.25) (layer "B.Cu") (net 1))
 (segment (start 134.7656 63.4206) (end 156.2894 63.4206) (width 0.25) (layer "B.Cu") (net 1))
 (segment (start 143.3651 26.67) (end 143.6102 26.4249) (width 0.25) (layer "B.Cu") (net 1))
 (segment (start 142.24 26.67) (end 143.3651 26.67) (width 0.25) (layer "B.Cu") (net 1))
 (segment (start 131.2774 59.9324) (end 134.7656 63.4206) (width 0.25) (layer "B.Cu") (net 1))
 (segment (start 161.4306 61.1638) (end 161.4306 60.2091) (width 0.25) (layer "F.Cu") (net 3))
 (via (at 161.4306 61.1638) (size 0.8) (drill 0.4) (layers "F.Cu" "B.Cu") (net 3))
 (segment (start 138.575 62.23) (end 142.24 62.23) (width 0.25) (layer "B.Cu") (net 3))
 (segment (start 142.24 62.23) (end 143.51 60.96) (width 0.25) (layer "B.Cu") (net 3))
 (segment (start 156.3305 60.96) (end 161.2268 60.96) (width 0.25) (layer "B.Cu") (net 3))
 (segment (start 161.2268 60.96) (end 161.4306 61.1638) (width 0.25) (layer "B.Cu") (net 3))
 (segment (start 143.51 60.96) (end 156.3305 60.96) (width 0.25) (layer "B.Cu") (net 3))
 (segment (start 156.3305 32.8995) (end 157.48 31.75) (width 0.25) (layer "B.Cu") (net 3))
 (segment (start 156.3305 60.96) (end 156.3305 32.8995) (width 0.25) (layer "B.Cu") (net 3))
 (segment (start 136.2774 59.9324) (end 138.575 62.23) (width 0.25) (layer "B.Cu") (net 3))
 (segment (start 169.5805 60.2091) (end 169.3169 60.4727) (width 0.25) (layer "F.Cu") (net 20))
 (segment (start 169.3169 60.4727) (end 168.6227 60.4727) (width 0.25) (layer "F.Cu") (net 20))
 (segment (start 170.8806 60.2091) (end 169.5805 60.2091) (width 0.25) (layer "F.Cu") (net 20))
 (via (at 168.6227 60.4727) (size 0.8) (drill 0.4) (layers "F.Cu" "B.Cu") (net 20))
 (segment (start 165.3 57.15) (end 168.6227 60.4727) (width 0.25) (layer "B.Cu") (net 20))
 (segment (start 157.48 57.15) (end 165.3 57.15) (width 0.25) (layer "B.Cu") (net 20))
 (segment (start 141.1006 32.279) (end 141.6968 32.8752) (width 0.25) (layer "F.Cu") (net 21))
 (segment (start 142.5402 32.8752) (end 143.7594 34.0944) (width 0.25) (layer "F.Cu") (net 21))
 (segment (start 141.6968 32.8752) (end 142.5402 32.8752) (width 0.25) (layer "F.Cu") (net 21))
 (segment (start 142.24 29.21) (end 141.1006 30.3494) (width 0.25) (layer "F.Cu") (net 21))
 (segment (start 154.9337 38.1) (end 157.9085 38.1) (width 0.25) (layer "F.Cu") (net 21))
 (segment (start 143.7594 34.0944) (end 150.9281 34.0944) (width 0.25) (layer "F.Cu") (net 21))
 (segment (start 141.1006 30.3494) (end 141.1006 32.279) (width 0.25) (layer "F.Cu") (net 21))
 (segment (start 157.9085 38.1) (end 168.5876 48.7791) (width 0.25) (layer "F.Cu") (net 21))
 (segment (start 150.9281 34.0944) (end 154.9337 38.1) (width 0.25) (layer "F.Cu") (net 21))
 (segment (start 168.5876 48.7791) (end 170.8806 48.7791) (width 0.25) (layer "F.Cu") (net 21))
 (segment (start 157.8759 35.56) (end 169.5805 47.2646) (width 0.25) (layer "F.Cu") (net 22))
 (segment (start 170.8806 47.5091) (end 169.5805 47.5091) (width 0.25) (layer "F.Cu") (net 22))
 (segment (start 169.5805 47.2646) (end 169.5805 47.5091) (width 0.25) (layer "F.Cu") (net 22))
 (segment (start 155.5886 35.56) (end 157.8759 35.56) (width 0.25) (layer "F.Cu") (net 22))
 (segment (start 142.24 31.75) (end 151.7786 31.75) (width 0.25) (layer "F.Cu") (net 22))
 (segment (start 151.7786 31.75) (end 155.5886 35.56) (width 0.25) (layer "F.Cu") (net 22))
 (segment (start 142.24 34.29) (end 141.1006 35.4294) (width 0.25) (layer "F.Cu") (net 24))
 (segment (start 148.6198 41.8592) (end 154.8895 48.1289) (width 0.25) (layer "F.Cu") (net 24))
 (segment (start 141.1006 37.3539) (end 141.8467 38.1) (width 0.25) (layer "F.Cu") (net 24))
 (segment (start 141.8467 38.1) (end 142.5686 38.1) (width 0.25) (layer "F.Cu") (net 24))
 (segment (start 159.5107 48.1289) (end 160.1305 47.5091) (width 0.25) (layer "F.Cu") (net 24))
 (segment (start 142.5686 38.1) (end 144.023 39.5544) (width 0.25) (layer "F.Cu") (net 24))
 (segment (start 144.9572 41.8592) (end 148.6198 41.8592) (width 0.25) (layer "F.Cu") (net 24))
 (segment (start 161.4306 47.5091) (end 160.1305 47.5091) (width 0.25) (layer "F.Cu") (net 24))
 (segment (start 141.1006 35.4294) (end 141.1006 37.3539) (width 0.25) (layer "F.Cu") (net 24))
 (segment (start 144.023 40.925) (end 144.9572 41.8592) (width 0.25) (layer "F.Cu") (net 24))
 (segment (start 144.023 39.5544) (end 144.023 40.925) (width 0.25) (layer "F.Cu") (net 24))
 (segment (start 154.8895 48.1289) (end 159.5107 48.1289) (width 0.25) (layer "F.Cu") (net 24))
 (segment (start 142.24 36.83) (end 144.7292 39.3192) (width 0.25) (layer "F.Cu") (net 23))
 (segment (start 153.6115 45.589) (end 159.4804 45.589) (width 0.25) (layer "F.Cu") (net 23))
 (segment (start 159.4804 45.589) (end 160.1305 46.2391) (width 0.25) (layer "F.Cu") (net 23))
 (segment (start 147.3417 39.3192) (end 153.6115 45.589) (width 0.25) (layer "F.Cu") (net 23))
 (segment (start 144.7292 39.3192) (end 147.3417 39.3192) (width 0.25) (layer "F.Cu") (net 23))
 (segment (start 161.4306 46.2391) (end 160.1305 46.2391) (width 0.25) (layer "F.Cu") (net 23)))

